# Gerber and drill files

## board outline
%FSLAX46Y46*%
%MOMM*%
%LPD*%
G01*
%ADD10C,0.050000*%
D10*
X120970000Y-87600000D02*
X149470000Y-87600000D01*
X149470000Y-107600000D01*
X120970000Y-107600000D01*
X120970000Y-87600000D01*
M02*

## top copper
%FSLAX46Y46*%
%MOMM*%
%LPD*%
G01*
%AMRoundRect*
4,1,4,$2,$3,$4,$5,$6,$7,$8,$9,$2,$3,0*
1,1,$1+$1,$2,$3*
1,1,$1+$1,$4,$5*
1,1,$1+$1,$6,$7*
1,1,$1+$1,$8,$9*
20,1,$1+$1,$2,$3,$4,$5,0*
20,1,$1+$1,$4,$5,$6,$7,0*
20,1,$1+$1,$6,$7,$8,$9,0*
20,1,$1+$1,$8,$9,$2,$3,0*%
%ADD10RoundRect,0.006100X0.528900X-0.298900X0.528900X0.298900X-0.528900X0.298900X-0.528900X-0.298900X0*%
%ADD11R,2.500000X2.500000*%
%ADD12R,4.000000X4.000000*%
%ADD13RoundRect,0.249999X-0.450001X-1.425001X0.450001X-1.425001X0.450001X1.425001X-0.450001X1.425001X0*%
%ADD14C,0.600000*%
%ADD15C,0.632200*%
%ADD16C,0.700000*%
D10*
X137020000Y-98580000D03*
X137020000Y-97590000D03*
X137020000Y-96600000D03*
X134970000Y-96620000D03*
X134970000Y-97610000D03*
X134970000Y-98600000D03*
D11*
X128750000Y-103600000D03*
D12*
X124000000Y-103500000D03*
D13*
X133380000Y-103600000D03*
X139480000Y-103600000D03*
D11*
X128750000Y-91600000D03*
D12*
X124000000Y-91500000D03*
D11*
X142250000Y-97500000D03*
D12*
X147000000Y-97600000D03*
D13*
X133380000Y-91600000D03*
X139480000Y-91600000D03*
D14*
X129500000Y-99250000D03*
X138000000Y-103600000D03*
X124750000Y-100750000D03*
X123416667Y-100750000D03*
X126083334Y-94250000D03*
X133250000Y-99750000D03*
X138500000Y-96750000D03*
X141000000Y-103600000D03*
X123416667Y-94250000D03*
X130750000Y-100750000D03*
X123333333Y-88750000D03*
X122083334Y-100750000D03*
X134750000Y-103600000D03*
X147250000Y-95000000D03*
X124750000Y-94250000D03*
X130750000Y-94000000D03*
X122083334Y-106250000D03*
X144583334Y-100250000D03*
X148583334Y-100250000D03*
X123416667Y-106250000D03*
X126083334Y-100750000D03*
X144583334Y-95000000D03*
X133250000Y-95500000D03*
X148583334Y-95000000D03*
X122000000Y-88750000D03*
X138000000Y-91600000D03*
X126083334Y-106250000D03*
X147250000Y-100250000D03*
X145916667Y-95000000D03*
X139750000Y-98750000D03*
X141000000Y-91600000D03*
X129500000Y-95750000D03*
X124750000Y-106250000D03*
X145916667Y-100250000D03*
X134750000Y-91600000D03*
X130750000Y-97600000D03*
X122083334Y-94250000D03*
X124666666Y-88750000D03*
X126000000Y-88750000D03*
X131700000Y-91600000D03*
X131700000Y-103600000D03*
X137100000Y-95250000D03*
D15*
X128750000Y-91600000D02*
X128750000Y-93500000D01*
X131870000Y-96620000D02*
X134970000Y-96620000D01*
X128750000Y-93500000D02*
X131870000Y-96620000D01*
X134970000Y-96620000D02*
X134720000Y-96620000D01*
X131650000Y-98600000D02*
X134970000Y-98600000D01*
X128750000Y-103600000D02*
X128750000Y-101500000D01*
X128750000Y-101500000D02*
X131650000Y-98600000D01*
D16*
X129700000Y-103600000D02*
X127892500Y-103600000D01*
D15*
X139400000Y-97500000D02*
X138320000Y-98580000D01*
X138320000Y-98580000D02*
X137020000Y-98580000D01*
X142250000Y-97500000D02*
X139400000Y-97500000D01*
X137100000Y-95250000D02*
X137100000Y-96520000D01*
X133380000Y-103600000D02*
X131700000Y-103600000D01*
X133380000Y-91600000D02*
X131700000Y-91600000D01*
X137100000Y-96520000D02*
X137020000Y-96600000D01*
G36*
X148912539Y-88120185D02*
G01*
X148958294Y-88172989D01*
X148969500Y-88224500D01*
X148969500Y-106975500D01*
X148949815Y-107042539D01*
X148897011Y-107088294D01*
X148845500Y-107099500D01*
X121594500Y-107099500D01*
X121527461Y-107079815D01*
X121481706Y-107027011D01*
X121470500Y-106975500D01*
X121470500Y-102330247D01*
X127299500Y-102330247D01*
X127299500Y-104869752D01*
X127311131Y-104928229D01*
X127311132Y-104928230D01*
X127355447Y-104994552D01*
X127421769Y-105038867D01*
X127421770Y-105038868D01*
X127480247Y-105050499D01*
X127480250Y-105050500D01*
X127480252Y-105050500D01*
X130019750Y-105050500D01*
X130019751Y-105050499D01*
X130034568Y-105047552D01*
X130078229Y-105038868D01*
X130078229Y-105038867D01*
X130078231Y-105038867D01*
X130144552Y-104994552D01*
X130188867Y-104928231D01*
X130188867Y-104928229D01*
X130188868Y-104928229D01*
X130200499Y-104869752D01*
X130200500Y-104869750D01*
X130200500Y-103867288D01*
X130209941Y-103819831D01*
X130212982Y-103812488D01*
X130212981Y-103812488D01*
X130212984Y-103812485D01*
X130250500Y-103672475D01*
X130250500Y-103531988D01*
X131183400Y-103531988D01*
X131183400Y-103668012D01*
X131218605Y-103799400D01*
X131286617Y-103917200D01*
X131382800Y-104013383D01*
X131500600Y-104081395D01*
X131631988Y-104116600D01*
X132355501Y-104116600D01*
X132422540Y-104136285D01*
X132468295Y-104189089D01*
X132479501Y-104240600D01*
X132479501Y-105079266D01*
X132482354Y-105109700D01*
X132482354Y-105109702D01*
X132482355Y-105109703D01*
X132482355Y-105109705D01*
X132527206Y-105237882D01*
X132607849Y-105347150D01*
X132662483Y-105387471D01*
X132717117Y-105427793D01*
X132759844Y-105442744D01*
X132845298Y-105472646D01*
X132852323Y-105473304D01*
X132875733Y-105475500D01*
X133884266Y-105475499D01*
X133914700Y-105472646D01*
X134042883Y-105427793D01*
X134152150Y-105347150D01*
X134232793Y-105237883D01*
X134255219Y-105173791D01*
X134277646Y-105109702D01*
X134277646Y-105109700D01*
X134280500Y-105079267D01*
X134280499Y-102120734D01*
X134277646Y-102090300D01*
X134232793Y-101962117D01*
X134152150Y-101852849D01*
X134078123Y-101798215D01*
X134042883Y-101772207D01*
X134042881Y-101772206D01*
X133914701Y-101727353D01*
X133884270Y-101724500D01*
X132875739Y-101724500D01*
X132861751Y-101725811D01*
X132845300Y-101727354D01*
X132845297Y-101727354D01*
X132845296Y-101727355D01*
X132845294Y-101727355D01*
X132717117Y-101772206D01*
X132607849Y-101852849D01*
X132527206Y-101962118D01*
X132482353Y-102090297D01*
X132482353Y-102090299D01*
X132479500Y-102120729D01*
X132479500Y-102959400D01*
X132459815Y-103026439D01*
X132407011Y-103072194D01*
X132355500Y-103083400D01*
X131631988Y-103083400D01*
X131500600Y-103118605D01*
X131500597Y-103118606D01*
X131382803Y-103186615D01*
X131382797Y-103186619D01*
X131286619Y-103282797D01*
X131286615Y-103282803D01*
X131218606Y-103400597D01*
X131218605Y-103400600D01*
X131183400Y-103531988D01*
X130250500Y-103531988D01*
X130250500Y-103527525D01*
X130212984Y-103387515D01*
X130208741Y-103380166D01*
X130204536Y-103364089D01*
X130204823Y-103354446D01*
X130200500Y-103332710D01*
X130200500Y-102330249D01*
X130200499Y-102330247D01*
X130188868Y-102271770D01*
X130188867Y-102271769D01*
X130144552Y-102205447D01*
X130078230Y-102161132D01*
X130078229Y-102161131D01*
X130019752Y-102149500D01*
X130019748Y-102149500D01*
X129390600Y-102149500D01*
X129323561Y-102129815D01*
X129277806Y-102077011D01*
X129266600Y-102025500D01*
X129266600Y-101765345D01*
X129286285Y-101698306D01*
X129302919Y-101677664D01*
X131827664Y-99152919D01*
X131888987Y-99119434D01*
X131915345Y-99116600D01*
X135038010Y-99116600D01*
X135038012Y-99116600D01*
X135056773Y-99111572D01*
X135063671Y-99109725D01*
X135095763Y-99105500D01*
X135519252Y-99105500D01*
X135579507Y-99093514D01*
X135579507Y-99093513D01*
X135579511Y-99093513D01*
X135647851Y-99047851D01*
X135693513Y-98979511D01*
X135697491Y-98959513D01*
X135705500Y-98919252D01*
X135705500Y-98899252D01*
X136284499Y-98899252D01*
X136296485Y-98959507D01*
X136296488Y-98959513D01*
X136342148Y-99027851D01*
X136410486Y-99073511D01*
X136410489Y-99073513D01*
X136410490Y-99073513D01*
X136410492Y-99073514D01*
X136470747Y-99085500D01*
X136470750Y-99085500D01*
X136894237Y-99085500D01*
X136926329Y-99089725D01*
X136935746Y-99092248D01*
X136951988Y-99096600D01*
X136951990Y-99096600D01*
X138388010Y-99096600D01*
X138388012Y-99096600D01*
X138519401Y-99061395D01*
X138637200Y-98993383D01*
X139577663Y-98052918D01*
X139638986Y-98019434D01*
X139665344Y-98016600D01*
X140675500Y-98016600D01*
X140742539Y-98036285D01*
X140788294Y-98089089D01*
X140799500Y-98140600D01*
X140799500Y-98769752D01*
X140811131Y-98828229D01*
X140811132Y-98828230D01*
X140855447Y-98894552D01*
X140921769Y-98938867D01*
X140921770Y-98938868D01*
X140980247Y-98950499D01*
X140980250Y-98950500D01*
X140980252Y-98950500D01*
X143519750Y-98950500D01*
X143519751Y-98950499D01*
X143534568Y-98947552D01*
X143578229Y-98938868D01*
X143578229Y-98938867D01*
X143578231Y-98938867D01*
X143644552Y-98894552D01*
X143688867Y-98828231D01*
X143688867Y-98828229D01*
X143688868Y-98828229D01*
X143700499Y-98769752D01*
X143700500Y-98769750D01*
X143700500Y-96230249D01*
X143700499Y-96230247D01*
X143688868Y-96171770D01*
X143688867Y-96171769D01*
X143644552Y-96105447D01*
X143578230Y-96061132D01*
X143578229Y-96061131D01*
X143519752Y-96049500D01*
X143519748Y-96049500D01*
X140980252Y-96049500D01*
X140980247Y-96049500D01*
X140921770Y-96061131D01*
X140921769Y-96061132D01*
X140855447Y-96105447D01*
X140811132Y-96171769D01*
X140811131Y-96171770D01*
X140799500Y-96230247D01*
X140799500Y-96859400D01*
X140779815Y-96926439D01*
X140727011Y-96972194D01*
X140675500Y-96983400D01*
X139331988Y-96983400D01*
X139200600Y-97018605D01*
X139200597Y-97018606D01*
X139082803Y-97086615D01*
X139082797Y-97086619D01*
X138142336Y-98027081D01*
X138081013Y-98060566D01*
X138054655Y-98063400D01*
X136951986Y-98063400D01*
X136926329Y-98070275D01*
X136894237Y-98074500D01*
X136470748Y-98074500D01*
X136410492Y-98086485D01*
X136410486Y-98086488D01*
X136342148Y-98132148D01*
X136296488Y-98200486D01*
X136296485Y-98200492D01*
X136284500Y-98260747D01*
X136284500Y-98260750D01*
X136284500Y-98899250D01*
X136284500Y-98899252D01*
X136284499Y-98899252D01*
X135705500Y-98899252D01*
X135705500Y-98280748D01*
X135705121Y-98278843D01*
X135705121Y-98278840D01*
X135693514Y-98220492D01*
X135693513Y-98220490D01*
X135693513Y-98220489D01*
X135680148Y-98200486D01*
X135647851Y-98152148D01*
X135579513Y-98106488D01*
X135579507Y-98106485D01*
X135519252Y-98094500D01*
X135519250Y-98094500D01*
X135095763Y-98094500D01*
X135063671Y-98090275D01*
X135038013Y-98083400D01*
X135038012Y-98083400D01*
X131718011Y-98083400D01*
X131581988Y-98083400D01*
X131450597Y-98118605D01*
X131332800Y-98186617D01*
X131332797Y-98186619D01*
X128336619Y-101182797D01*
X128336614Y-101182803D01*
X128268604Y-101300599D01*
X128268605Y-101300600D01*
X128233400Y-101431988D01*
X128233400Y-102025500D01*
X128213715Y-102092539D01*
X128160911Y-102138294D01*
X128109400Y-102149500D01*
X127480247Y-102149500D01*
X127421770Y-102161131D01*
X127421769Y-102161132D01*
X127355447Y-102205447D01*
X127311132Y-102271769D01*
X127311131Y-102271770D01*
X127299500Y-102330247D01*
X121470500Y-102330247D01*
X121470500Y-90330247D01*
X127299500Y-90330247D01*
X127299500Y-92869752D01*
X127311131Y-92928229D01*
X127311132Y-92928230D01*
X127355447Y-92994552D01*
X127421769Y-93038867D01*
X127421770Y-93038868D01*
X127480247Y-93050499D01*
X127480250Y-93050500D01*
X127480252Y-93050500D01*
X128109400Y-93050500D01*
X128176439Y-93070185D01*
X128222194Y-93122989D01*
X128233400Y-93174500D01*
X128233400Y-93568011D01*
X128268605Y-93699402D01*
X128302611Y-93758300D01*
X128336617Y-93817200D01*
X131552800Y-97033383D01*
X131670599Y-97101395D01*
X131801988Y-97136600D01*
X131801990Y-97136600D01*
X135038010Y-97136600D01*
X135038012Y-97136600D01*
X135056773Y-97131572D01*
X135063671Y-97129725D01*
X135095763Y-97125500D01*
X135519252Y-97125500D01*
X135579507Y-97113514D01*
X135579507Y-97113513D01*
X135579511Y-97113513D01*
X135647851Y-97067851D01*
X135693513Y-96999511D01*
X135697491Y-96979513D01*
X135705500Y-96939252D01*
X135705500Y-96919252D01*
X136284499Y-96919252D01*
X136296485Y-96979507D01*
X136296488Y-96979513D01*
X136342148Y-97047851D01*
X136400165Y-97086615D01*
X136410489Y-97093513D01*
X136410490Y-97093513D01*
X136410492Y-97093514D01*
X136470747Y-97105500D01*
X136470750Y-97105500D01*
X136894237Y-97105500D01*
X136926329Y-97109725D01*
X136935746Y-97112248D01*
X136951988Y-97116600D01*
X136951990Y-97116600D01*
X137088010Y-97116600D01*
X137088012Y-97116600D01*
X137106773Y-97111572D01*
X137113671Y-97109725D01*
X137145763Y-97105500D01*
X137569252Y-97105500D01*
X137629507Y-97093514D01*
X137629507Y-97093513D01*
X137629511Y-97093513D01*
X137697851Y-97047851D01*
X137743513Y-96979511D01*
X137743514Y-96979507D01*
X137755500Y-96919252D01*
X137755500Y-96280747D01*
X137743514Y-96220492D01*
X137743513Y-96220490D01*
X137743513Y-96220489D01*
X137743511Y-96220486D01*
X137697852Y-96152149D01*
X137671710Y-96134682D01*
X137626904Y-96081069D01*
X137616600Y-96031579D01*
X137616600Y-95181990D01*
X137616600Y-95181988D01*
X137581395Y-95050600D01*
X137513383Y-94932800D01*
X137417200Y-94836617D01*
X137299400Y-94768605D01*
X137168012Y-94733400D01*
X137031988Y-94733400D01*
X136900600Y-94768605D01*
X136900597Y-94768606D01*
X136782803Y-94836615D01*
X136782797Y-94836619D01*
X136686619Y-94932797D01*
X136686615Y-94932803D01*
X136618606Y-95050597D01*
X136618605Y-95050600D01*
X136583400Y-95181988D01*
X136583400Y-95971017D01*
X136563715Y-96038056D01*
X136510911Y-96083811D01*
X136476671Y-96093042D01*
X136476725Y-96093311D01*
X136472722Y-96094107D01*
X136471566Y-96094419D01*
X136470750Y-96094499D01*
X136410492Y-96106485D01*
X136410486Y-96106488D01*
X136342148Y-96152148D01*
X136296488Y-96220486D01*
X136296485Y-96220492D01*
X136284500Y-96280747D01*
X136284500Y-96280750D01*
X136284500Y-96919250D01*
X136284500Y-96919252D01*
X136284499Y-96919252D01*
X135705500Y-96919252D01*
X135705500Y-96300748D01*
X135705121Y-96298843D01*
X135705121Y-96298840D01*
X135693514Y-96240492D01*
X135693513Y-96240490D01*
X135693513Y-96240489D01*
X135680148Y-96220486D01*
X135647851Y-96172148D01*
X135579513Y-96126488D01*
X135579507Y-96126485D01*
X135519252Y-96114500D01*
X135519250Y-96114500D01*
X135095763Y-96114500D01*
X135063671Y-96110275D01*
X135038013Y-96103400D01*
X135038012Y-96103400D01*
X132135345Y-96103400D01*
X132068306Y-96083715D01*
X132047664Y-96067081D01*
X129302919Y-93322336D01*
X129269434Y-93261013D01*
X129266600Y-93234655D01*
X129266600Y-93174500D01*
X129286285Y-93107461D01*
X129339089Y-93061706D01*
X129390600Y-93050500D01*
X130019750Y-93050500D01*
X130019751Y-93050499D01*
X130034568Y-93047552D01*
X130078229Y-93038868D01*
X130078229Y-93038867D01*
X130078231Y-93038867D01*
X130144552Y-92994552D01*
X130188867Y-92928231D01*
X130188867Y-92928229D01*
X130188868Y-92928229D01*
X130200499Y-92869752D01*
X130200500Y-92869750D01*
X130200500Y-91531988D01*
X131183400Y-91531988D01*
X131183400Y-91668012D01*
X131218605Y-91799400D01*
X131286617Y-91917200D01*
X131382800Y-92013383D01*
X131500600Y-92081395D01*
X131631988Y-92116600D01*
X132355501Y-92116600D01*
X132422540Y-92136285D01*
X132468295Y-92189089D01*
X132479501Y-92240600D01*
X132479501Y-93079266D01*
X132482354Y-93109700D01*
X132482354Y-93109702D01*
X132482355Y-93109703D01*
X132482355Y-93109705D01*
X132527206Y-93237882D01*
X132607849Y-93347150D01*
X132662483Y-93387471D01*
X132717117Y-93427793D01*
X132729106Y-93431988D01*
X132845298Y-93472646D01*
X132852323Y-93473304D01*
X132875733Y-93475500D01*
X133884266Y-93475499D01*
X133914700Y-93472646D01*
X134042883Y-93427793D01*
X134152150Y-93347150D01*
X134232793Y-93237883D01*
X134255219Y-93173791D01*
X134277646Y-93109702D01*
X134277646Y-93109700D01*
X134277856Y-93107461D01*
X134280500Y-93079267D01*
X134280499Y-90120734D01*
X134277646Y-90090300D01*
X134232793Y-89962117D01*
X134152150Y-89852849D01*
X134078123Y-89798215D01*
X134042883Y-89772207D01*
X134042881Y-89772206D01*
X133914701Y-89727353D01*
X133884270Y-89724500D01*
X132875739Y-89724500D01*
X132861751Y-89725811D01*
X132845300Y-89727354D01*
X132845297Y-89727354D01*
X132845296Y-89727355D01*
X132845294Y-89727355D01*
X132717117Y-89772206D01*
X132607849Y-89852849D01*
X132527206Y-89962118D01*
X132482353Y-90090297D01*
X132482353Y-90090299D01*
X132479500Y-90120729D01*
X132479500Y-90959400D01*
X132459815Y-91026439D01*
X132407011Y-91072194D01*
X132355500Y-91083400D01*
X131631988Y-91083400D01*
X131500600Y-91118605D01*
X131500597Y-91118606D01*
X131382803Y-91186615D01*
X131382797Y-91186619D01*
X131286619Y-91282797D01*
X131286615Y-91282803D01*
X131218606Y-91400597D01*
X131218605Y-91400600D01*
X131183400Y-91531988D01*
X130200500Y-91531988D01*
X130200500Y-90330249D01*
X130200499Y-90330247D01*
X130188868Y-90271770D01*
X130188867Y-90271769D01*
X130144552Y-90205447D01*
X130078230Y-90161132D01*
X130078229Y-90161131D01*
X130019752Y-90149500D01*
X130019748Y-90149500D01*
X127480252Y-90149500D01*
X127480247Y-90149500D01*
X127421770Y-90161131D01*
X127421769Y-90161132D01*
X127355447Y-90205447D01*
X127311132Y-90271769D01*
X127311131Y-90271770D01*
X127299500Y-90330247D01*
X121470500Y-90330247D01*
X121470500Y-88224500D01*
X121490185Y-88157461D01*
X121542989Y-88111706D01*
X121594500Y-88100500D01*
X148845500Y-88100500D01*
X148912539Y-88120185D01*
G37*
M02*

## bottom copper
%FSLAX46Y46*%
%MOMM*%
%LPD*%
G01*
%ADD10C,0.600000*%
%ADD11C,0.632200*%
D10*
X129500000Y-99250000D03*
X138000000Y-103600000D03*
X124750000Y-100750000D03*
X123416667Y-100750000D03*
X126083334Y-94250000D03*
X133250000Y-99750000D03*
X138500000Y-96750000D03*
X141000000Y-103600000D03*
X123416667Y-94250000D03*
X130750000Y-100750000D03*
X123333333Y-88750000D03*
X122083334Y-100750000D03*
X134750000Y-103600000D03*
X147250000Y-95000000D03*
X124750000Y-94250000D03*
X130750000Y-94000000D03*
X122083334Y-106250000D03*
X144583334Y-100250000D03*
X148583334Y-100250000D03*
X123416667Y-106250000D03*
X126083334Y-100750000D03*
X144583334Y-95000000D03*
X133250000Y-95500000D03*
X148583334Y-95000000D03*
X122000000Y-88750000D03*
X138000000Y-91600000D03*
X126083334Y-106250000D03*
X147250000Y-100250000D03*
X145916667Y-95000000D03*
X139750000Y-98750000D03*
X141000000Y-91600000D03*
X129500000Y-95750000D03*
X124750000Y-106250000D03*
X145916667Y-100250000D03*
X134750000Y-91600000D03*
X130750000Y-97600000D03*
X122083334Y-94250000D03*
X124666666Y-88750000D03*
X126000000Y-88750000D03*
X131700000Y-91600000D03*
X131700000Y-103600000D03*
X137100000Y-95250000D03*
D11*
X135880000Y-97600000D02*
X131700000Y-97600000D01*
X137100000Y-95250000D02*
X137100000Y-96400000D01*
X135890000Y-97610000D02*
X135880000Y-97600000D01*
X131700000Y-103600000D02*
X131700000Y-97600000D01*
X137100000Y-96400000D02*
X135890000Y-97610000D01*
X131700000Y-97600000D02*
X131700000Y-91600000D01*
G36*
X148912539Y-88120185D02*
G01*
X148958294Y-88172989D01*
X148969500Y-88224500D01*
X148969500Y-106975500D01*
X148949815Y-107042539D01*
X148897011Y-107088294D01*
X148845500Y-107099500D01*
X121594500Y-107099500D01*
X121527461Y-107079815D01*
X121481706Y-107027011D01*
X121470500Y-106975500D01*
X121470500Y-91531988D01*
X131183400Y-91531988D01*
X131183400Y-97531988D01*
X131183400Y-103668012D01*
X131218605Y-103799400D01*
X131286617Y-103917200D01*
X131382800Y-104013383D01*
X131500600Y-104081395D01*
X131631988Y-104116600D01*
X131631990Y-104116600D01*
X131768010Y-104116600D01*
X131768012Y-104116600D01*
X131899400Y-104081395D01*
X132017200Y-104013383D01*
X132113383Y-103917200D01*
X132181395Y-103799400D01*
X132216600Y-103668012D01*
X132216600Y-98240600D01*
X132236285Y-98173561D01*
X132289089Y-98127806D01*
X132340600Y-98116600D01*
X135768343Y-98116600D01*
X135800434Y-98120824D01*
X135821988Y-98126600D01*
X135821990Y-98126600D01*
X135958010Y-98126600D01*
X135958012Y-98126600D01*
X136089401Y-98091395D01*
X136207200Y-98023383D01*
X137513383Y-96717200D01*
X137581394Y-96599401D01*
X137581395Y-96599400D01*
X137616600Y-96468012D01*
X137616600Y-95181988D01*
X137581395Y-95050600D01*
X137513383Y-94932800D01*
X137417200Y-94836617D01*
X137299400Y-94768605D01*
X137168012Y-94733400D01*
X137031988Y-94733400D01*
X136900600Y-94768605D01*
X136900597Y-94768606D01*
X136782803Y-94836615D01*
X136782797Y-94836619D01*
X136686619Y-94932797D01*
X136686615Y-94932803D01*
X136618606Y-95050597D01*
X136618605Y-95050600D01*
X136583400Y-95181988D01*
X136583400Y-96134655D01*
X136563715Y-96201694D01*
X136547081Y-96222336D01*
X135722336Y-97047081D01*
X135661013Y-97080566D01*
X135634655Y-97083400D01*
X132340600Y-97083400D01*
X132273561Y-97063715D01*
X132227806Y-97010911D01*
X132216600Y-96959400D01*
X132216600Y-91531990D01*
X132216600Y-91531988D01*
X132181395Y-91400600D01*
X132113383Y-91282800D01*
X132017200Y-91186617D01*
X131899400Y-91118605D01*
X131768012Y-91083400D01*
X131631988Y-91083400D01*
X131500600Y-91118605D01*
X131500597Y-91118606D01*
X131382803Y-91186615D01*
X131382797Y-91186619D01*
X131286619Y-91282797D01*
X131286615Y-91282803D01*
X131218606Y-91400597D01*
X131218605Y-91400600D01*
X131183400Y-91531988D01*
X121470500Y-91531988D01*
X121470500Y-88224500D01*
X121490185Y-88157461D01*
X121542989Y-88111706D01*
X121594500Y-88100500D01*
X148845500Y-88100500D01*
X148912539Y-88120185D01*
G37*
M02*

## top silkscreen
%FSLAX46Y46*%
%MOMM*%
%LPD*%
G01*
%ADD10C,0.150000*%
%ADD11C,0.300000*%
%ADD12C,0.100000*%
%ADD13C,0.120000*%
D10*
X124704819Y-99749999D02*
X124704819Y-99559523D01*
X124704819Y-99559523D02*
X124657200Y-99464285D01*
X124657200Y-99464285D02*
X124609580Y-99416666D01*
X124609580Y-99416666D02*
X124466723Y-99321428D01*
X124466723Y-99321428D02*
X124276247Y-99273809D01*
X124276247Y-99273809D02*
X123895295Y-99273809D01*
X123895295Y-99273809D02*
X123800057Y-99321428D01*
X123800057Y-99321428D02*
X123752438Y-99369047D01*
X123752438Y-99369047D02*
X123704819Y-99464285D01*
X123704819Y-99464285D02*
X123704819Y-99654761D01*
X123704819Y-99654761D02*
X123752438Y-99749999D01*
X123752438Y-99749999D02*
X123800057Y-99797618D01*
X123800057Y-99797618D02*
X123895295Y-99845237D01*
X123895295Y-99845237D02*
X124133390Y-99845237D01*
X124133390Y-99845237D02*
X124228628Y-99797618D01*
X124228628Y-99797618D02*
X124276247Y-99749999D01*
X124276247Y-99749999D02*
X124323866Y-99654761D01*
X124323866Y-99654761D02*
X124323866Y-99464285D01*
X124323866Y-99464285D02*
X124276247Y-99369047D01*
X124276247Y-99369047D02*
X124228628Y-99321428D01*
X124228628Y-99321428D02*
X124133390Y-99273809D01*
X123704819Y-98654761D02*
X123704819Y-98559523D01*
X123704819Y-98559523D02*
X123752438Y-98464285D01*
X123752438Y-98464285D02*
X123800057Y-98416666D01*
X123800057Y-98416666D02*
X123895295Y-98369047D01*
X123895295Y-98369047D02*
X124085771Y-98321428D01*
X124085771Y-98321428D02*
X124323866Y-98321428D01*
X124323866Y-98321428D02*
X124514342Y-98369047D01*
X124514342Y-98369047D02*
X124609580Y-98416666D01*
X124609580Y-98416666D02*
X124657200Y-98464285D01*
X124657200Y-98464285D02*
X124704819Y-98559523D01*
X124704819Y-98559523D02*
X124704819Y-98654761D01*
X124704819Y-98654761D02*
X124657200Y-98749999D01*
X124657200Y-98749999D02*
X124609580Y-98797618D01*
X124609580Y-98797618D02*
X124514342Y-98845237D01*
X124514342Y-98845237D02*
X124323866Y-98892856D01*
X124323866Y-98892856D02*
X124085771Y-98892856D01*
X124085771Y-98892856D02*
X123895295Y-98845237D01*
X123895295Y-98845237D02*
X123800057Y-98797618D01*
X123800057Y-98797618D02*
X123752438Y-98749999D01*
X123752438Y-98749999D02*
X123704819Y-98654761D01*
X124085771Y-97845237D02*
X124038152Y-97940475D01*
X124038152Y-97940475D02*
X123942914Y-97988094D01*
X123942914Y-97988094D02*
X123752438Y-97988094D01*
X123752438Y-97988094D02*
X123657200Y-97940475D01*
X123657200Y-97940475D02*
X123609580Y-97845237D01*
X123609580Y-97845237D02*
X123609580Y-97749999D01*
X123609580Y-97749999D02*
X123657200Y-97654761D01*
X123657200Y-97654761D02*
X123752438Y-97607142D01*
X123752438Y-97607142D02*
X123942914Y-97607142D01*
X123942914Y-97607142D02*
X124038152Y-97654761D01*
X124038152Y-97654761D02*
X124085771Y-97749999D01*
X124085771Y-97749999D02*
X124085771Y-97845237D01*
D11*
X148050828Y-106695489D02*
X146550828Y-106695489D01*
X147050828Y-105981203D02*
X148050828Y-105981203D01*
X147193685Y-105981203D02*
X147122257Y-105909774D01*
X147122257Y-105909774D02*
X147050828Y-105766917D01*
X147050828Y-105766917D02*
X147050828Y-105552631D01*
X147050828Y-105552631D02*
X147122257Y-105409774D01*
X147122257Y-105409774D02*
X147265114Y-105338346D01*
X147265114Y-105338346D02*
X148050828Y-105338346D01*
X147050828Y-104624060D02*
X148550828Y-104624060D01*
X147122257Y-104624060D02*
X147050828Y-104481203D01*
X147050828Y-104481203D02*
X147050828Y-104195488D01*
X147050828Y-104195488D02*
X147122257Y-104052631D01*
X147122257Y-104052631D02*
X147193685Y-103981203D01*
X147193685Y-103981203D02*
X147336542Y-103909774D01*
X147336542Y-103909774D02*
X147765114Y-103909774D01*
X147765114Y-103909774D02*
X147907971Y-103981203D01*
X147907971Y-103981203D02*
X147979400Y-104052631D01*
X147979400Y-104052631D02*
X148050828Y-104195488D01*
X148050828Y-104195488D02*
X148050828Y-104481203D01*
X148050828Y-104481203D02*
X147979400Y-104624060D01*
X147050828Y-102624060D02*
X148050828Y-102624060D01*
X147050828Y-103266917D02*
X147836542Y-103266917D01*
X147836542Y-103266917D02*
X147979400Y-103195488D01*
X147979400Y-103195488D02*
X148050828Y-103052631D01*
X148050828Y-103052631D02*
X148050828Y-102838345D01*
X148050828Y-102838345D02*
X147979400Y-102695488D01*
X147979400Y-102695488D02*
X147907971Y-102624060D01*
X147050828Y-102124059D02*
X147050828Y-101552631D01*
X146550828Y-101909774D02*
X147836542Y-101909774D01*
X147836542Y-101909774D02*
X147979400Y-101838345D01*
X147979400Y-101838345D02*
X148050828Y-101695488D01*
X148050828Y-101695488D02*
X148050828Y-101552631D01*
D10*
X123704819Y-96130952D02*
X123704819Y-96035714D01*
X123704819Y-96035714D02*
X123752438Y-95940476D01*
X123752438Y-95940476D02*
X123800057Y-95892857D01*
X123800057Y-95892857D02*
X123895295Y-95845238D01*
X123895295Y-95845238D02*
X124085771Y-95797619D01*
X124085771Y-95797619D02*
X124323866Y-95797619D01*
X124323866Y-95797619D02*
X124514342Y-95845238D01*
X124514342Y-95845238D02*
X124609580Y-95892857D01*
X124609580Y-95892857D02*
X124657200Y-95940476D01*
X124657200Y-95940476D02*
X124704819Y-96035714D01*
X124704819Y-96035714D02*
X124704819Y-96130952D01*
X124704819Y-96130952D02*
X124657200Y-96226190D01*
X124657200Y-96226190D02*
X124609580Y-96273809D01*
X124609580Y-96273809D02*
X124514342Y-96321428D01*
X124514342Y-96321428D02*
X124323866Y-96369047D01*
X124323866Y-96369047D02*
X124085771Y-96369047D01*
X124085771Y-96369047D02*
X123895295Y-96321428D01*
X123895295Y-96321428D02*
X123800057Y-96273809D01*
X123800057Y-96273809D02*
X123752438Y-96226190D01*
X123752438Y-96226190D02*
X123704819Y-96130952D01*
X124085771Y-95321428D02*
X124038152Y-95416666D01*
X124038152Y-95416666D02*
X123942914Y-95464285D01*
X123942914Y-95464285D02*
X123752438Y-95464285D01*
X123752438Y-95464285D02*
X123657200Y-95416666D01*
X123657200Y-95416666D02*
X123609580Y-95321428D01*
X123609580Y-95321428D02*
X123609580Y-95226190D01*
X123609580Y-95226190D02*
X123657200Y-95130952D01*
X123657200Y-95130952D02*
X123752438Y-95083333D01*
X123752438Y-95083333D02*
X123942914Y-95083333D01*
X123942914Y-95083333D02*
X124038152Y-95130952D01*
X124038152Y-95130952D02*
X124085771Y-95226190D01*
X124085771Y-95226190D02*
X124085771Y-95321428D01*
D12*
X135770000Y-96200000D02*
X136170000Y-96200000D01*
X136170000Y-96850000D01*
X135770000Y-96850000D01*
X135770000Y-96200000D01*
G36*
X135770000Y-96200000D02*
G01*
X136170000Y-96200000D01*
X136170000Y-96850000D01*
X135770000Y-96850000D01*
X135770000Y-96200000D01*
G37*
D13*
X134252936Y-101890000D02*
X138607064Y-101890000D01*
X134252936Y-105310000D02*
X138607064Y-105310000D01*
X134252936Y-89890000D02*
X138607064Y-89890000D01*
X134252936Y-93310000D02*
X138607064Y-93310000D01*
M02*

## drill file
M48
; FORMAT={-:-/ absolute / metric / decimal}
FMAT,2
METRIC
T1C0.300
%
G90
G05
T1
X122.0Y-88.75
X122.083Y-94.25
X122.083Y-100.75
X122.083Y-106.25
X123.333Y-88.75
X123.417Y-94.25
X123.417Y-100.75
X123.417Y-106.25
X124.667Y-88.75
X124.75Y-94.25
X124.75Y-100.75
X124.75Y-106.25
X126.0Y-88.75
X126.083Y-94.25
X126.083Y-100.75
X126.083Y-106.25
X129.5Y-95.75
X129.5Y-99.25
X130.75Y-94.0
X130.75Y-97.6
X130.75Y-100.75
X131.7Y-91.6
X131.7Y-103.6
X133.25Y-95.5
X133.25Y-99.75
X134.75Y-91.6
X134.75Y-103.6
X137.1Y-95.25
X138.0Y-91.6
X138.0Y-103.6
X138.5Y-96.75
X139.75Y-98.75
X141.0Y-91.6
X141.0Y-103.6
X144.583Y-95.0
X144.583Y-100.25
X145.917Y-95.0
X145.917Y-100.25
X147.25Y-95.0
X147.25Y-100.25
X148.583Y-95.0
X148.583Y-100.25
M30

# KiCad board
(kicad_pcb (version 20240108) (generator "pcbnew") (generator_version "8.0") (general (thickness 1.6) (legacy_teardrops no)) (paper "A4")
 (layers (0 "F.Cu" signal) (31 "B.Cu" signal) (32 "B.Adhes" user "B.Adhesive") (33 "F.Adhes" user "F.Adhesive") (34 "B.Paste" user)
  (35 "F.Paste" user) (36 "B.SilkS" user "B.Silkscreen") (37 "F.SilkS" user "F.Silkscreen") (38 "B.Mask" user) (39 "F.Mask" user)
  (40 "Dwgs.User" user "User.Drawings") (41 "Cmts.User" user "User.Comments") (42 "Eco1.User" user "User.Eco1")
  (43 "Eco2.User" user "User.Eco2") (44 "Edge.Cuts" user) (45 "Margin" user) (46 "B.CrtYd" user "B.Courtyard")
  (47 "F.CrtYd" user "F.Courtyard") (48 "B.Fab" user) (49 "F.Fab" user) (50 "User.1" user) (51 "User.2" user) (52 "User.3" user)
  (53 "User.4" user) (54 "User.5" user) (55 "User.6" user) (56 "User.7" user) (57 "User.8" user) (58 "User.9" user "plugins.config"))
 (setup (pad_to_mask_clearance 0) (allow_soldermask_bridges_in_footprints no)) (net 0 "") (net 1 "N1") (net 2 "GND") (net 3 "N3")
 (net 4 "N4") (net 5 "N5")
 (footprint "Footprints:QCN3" (layer "F.Cu") (at 136.97 97.6 90)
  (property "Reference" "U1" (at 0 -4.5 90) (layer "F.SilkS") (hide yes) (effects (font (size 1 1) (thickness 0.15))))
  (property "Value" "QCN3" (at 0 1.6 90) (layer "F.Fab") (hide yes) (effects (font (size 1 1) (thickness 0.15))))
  (fp_rect (start 0.75 -1.2) (end 1.4 -0.8) (stroke (width 0.1) (type solid)) (fill solid) (layer "F.SilkS"))
  (pad "1" smd roundrect (at -0.98 0.05 90) (size 0.61 1.07) (layers "F.Cu" "F.Paste" "F.Mask") (roundrect_rratio 0.01) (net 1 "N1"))
  (pad "2" smd roundrect (at 0.01 0.05 90) (size 0.61 1.07) (layers "F.Cu" "F.Paste" "F.Mask") (roundrect_rratio 0.01) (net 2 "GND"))
  (pad "3" smd roundrect (at 1 0.05 90) (size 0.61 1.07) (layers "F.Cu" "F.Paste" "F.Mask") (roundrect_rratio 0.01) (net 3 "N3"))
  (pad "4" smd roundrect (at 0.98 -2 90) (size 0.61 1.07) (layers "F.Cu" "F.Paste" "F.Mask") (roundrect_rratio 0.01) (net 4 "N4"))
  (pad "5" smd roundrect (at -0.01 -2 90) (size 0.61 1.07) (layers "F.Cu" "F.Paste" "F.Mask") (roundrect_rratio 0.01) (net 2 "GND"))
  (pad "6" smd roundrect (at -1 -2 90) (size 0.61 1.07) (layers "F.Cu" "F.Paste" "F.Mask") (roundrect_rratio 0.01) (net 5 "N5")))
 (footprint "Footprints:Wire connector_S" (layer "F.Cu") (at 128.5 103.6 180)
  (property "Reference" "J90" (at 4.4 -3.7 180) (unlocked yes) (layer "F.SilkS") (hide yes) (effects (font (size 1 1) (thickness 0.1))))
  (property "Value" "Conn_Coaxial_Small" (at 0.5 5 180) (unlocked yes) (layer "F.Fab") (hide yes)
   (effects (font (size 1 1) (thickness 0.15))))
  (pad "1" smd rect (at -0.25 0 90) (size 2.5 2.5) (layers "F.Cu" "F.Paste" "F.Mask") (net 5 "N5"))
  (pad "2" smd rect (at 4.5 0.1 90) (size 4 4) (layers "F.Cu" "F.Paste" "F.Mask") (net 2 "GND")))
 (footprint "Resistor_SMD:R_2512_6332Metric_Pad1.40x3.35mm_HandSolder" (layer "F.Cu") (at 136.43 103.6)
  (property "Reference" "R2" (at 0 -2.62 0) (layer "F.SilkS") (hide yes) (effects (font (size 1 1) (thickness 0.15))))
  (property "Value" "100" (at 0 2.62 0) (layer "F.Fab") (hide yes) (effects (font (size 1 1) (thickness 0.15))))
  (fp_line (start -2.177064 -1.71) (end 2.177064 -1.71) (stroke (width 0.12) (type solid)) (layer "F.SilkS"))
  (fp_line (start -2.177064 1.71) (end 2.177064 1.71) (stroke (width 0.12) (type solid)) (layer "F.SilkS"))
  (pad "1" smd roundrect (at -3.05 0) (size 1.4 3.35) (layers "F.Cu" "F.Paste" "F.Mask") (roundrect_rratio 0.178571) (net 3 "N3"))
  (pad "2" smd roundrect (at 3.05 0) (size 1.4 3.35) (layers "F.Cu" "F.Paste" "F.Mask") (roundrect_rratio 0.178571) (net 2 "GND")))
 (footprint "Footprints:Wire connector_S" (layer "F.Cu") (at 128.5 91.6 180)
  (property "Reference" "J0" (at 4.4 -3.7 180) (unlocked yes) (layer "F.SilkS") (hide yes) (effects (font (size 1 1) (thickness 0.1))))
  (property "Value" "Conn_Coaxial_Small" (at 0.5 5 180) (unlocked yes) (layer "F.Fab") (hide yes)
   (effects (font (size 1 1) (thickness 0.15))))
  (pad "1" smd rect (at -0.25 0 90) (size 2.5 2.5) (layers "F.Cu" "F.Paste" "F.Mask") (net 4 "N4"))
  (pad "2" smd rect (at 4.5 0.1 90) (size 4 4) (layers "F.Cu" "F.Paste" "F.Mask") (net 2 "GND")))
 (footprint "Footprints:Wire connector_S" (layer "F.Cu") (at 142.5 97.5)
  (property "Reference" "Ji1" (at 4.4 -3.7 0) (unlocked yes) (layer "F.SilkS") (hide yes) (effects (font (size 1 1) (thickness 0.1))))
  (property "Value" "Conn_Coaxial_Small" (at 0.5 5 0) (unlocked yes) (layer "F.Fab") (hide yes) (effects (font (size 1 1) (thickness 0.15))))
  (pad "1" smd rect (at -0.25 0 270) (size 2.5 2.5) (layers "F.Cu" "F.Paste" "F.Mask") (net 1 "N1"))
  (pad "2" smd rect (at 4.5 0.1 270) (size 4 4) (layers "F.Cu" "F.Paste" "F.Mask") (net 2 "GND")))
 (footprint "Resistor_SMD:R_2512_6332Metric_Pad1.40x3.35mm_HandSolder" (layer "F.Cu") (at 136.43 91.6)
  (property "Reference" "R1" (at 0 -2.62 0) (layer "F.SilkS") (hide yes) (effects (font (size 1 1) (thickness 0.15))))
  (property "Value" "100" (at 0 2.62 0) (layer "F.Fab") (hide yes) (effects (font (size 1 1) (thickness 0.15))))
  (fp_line (start -2.177064 -1.71) (end 2.177064 -1.71) (stroke (width 0.12) (type solid)) (layer "F.SilkS"))
  (fp_line (start -2.177064 1.71) (end 2.177064 1.71) (stroke (width 0.12) (type solid)) (layer "F.SilkS"))
  (pad "1" smd roundrect (at -3.05 0) (size 1.4 3.35) (layers "F.Cu" "F.Paste" "F.Mask") (roundrect_rratio 0.178571) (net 3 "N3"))
  (pad "2" smd roundrect (at 3.05 0) (size 1.4 3.35) (layers "F.Cu" "F.Paste" "F.Mask") (roundrect_rratio 0.178571) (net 2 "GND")))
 (gr_rect (start 120.97 87.6) (end 149.47 107.6) (stroke (width 0.05) (type default)) (fill none) (layer "Edge.Cuts"))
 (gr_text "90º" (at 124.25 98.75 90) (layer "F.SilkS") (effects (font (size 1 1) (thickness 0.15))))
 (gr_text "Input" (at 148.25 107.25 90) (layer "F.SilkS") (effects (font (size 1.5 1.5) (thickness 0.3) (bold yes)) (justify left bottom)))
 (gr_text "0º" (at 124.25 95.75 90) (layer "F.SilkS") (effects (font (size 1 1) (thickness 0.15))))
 (via (at 129.5 99.25) (size 0.6) (drill 0.3) (layers "F.Cu" "B.Cu") (free yes) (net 2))
 (via (at 138 103.6) (size 0.6) (drill 0.3) (layers "F.Cu" "B.Cu") (free yes) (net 2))
 (via (at 124.75 100.75) (size 0.6) (drill 0.3) (layers "F.Cu" "B.Cu") (free yes) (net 2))
 (via (at 123.416667 100.75) (size 0.6) (drill 0.3) (layers "F.Cu" "B.Cu") (free yes) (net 2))
 (via (at 126.083334 94.25) (size 0.6) (drill 0.3) (layers "F.Cu" "B.Cu") (free yes) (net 2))
 (via (at 133.25 99.75) (size 0.6) (drill 0.3) (layers "F.Cu" "B.Cu") (free yes) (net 2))
 (via (at 138.5 96.75) (size 0.6) (drill 0.3) (layers "F.Cu" "B.Cu") (free yes) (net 2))
 (via (at 141 103.6) (size 0.6) (drill 0.3) (layers "F.Cu" "B.Cu") (free yes) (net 2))
 (via (at 123.416667 94.25) (size 0.6) (drill 0.3) (layers "F.Cu" "B.Cu") (free yes) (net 2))
 (via (at 130.75 100.75) (size 0.6) (drill 0.3) (layers "F.Cu" "B.Cu") (free yes) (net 2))
 (via (at 123.333333 88.75) (size 0.6) (drill 0.3) (layers "F.Cu" "B.Cu") (free yes) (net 2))
 (via (at 122.083334 100.75) (size 0.6) (drill 0.3) (layers "F.Cu" "B.Cu") (free yes) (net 2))
 (via (at 134.75 103.6) (size 0.6) (drill 0.3) (layers "F.Cu" "B.Cu") (free yes) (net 2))
 (via (at 147.25 95) (size 0.6) (drill 0.3) (layers "F.Cu" "B.Cu") (free yes) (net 2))
 (via (at 124.75 94.25) (size 0.6) (drill 0.3) (layers "F.Cu" "B.Cu") (free yes) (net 2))
 (via (at 130.75 94) (size 0.6) (drill 0.3) (layers "F.Cu" "B.Cu") (free yes) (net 2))
 (via (at 122.083334 106.25) (size 0.6) (drill 0.3) (layers "F.Cu" "B.Cu") (free yes) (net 2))
 (via (at 144.583334 100.25) (size 0.6) (drill 0.3) (layers "F.Cu" "B.Cu") (free yes) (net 2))
 (via (at 148.583334 100.25) (size 0.6) (drill 0.3) (layers "F.Cu" "B.Cu") (free yes) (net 2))
 (via (at 123.416667 106.25) (size 0.6) (drill 0.3) (layers "F.Cu" "B.Cu") (free yes) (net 2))
 (via (at 126.083334 100.75) (size 0.6) (drill 0.3) (layers "F.Cu" "B.Cu") (free yes) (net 2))
 (via (at 144.583334 95) (size 0.6) (drill 0.3) (layers "F.Cu" "B.Cu") (free yes) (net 2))
 (via (at 133.25 95.5) (size 0.6) (drill 0.3) (layers "F.Cu" "B.Cu") (free yes) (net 2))
 (via (at 148.583334 95) (size 0.6) (drill 0.3) (layers "F.Cu" "B.Cu") (free yes) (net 2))
 (via (at 122 88.75) (size 0.6) (drill 0.3) (layers "F.Cu" "B.Cu") (free yes) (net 2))
 (via (at 138 91.6) (size 0.6) (drill 0.3) (layers "F.Cu" "B.Cu") (free yes) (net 2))
 (via (at 126.083334 106.25) (size 0.6) (drill 0.3) (layers "F.Cu" "B.Cu") (free yes) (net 2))
 (via (at 147.25 100.25) (size 0.6) (drill 0.3) (layers "F.Cu" "B.Cu") (free yes) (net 2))
 (via (at 145.916667 95) (size 0.6) (drill 0.3) (layers "F.Cu" "B.Cu") (free yes) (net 2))
 (via (at 139.75 98.75) (size 0.6) (drill 0.3) (layers "F.Cu" "B.Cu") (free yes) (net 2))
 (via (at 141 91.6) (size 0.6) (drill 0.3) (layers "F.Cu" "B.Cu") (free yes) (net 2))
 (via (at 129.5 95.75) (size 0.6) (drill 0.3) (layers "F.Cu" "B.Cu") (free yes) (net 2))
 (via (at 124.75 106.25) (size 0.6) (drill 0.3) (layers "F.Cu" "B.Cu") (free yes) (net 2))
 (via (at 145.916667 100.25) (size 0.6) (drill 0.3) (layers "F.Cu" "B.Cu") (free yes) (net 2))
 (via (at 134.75 91.6) (size 0.6) (drill 0.3) (layers "F.Cu" "B.Cu") (free yes) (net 2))
 (via (at 130.75 97.6) (size 0.6) (drill 0.3) (layers "F.Cu" "B.Cu") (free yes) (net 2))
 (via (at 122.083334 94.25) (size 0.6) (drill 0.3) (layers "F.Cu" "B.Cu") (free yes) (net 2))
 (via (at 124.666666 88.75) (size 0.6) (drill 0.3) (layers "F.Cu" "B.Cu") (free yes) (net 2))
 (via (at 126 88.75) (size 0.6) (drill 0.3) (layers "F.Cu" "B.Cu") (free yes) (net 2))
 (segment (start 128.75 91.6) (end 128.75 93.5) (width 0.6322) (layer "F.Cu") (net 4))
 (segment (start 131.87 96.62) (end 134.97 96.62) (width 0.6322) (layer "F.Cu") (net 4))
 (segment (start 128.75 93.5) (end 131.87 96.62) (width 0.6322) (layer "F.Cu") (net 4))
 (segment (start 134.97 96.62) (end 134.72 96.62) (width 0.6322) (layer "F.Cu") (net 4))
 (segment (start 131.65 98.6) (end 134.97 98.6) (width 0.6322) (layer "F.Cu") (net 5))
 (segment (start 128.75 103.6) (end 128.75 101.5) (width 0.6322) (layer "F.Cu") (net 5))
 (segment (start 128.75 101.5) (end 131.65 98.6) (width 0.6322) (layer "F.Cu") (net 5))
 (segment (start 129.7 103.6) (end 127.8925 103.6) (width 0.7) (layer "F.Cu") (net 5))
 (segment (start 139.4 97.5) (end 138.32 98.58) (width 0.6322) (layer "F.Cu") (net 1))
 (segment (start 138.32 98.58) (end 137.02 98.58) (width 0.6322) (layer "F.Cu") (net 1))
 (segment (start 142.25 97.5) (end 139.4 97.5) (width 0.6322) (layer "F.Cu") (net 1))
 (segment (start 137.1 95.25) (end 137.1 96.52) (width 0.6322) (layer "F.Cu") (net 3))
 (segment (start 133.38 103.6) (end 131.7 103.6) (width 0.6322) (layer "F.Cu") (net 3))
 (segment (start 133.38 91.6) (end 131.7 91.6) (width 0.6322) (layer "F.Cu") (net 3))
 (segment (start 137.1 96.52) (end 137.02 96.6) (width 0.6322) (layer "F.Cu") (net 3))
 (via (at 131.7 91.6) (size 0.6) (drill 0.3) (layers "F.Cu" "B.Cu") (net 3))
 (via (at 131.7 103.6) (size 0.6) (drill 0.3) (layers "F.Cu" "B.Cu") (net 3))
 (via (at 137.1 95.25) (size 0.6) (drill 0.3) (layers "F.Cu" "B.Cu") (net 3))
 (segment (start 135.88 97.6) (end 131.7 97.6) (width 0.6322) (layer "B.Cu") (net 3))
 (segment (start 137.1 95.25) (end 137.1 96.4) (width 0.6322) (layer "B.Cu") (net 3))
 (segment (start 135.89 97.61) (end 135.88 97.6) (width 0.6322) (layer "B.Cu") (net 3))
 (segment (start 131.7 103.6) (end 131.7 97.6) (width 0.6322) (layer "B.Cu") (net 3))
 (segment (start 137.1 96.4) (end 135.89 97.61) (width 0.6322) (layer "B.Cu") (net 3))
 (segment (start 131.7 97.6) (end 131.7 91.6) (width 0.6322) (layer "B.Cu") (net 3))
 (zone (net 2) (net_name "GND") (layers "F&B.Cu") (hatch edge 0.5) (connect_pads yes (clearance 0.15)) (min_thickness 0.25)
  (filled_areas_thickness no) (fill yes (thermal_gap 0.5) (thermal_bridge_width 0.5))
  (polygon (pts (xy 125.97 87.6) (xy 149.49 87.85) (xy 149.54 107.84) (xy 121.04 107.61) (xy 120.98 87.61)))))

